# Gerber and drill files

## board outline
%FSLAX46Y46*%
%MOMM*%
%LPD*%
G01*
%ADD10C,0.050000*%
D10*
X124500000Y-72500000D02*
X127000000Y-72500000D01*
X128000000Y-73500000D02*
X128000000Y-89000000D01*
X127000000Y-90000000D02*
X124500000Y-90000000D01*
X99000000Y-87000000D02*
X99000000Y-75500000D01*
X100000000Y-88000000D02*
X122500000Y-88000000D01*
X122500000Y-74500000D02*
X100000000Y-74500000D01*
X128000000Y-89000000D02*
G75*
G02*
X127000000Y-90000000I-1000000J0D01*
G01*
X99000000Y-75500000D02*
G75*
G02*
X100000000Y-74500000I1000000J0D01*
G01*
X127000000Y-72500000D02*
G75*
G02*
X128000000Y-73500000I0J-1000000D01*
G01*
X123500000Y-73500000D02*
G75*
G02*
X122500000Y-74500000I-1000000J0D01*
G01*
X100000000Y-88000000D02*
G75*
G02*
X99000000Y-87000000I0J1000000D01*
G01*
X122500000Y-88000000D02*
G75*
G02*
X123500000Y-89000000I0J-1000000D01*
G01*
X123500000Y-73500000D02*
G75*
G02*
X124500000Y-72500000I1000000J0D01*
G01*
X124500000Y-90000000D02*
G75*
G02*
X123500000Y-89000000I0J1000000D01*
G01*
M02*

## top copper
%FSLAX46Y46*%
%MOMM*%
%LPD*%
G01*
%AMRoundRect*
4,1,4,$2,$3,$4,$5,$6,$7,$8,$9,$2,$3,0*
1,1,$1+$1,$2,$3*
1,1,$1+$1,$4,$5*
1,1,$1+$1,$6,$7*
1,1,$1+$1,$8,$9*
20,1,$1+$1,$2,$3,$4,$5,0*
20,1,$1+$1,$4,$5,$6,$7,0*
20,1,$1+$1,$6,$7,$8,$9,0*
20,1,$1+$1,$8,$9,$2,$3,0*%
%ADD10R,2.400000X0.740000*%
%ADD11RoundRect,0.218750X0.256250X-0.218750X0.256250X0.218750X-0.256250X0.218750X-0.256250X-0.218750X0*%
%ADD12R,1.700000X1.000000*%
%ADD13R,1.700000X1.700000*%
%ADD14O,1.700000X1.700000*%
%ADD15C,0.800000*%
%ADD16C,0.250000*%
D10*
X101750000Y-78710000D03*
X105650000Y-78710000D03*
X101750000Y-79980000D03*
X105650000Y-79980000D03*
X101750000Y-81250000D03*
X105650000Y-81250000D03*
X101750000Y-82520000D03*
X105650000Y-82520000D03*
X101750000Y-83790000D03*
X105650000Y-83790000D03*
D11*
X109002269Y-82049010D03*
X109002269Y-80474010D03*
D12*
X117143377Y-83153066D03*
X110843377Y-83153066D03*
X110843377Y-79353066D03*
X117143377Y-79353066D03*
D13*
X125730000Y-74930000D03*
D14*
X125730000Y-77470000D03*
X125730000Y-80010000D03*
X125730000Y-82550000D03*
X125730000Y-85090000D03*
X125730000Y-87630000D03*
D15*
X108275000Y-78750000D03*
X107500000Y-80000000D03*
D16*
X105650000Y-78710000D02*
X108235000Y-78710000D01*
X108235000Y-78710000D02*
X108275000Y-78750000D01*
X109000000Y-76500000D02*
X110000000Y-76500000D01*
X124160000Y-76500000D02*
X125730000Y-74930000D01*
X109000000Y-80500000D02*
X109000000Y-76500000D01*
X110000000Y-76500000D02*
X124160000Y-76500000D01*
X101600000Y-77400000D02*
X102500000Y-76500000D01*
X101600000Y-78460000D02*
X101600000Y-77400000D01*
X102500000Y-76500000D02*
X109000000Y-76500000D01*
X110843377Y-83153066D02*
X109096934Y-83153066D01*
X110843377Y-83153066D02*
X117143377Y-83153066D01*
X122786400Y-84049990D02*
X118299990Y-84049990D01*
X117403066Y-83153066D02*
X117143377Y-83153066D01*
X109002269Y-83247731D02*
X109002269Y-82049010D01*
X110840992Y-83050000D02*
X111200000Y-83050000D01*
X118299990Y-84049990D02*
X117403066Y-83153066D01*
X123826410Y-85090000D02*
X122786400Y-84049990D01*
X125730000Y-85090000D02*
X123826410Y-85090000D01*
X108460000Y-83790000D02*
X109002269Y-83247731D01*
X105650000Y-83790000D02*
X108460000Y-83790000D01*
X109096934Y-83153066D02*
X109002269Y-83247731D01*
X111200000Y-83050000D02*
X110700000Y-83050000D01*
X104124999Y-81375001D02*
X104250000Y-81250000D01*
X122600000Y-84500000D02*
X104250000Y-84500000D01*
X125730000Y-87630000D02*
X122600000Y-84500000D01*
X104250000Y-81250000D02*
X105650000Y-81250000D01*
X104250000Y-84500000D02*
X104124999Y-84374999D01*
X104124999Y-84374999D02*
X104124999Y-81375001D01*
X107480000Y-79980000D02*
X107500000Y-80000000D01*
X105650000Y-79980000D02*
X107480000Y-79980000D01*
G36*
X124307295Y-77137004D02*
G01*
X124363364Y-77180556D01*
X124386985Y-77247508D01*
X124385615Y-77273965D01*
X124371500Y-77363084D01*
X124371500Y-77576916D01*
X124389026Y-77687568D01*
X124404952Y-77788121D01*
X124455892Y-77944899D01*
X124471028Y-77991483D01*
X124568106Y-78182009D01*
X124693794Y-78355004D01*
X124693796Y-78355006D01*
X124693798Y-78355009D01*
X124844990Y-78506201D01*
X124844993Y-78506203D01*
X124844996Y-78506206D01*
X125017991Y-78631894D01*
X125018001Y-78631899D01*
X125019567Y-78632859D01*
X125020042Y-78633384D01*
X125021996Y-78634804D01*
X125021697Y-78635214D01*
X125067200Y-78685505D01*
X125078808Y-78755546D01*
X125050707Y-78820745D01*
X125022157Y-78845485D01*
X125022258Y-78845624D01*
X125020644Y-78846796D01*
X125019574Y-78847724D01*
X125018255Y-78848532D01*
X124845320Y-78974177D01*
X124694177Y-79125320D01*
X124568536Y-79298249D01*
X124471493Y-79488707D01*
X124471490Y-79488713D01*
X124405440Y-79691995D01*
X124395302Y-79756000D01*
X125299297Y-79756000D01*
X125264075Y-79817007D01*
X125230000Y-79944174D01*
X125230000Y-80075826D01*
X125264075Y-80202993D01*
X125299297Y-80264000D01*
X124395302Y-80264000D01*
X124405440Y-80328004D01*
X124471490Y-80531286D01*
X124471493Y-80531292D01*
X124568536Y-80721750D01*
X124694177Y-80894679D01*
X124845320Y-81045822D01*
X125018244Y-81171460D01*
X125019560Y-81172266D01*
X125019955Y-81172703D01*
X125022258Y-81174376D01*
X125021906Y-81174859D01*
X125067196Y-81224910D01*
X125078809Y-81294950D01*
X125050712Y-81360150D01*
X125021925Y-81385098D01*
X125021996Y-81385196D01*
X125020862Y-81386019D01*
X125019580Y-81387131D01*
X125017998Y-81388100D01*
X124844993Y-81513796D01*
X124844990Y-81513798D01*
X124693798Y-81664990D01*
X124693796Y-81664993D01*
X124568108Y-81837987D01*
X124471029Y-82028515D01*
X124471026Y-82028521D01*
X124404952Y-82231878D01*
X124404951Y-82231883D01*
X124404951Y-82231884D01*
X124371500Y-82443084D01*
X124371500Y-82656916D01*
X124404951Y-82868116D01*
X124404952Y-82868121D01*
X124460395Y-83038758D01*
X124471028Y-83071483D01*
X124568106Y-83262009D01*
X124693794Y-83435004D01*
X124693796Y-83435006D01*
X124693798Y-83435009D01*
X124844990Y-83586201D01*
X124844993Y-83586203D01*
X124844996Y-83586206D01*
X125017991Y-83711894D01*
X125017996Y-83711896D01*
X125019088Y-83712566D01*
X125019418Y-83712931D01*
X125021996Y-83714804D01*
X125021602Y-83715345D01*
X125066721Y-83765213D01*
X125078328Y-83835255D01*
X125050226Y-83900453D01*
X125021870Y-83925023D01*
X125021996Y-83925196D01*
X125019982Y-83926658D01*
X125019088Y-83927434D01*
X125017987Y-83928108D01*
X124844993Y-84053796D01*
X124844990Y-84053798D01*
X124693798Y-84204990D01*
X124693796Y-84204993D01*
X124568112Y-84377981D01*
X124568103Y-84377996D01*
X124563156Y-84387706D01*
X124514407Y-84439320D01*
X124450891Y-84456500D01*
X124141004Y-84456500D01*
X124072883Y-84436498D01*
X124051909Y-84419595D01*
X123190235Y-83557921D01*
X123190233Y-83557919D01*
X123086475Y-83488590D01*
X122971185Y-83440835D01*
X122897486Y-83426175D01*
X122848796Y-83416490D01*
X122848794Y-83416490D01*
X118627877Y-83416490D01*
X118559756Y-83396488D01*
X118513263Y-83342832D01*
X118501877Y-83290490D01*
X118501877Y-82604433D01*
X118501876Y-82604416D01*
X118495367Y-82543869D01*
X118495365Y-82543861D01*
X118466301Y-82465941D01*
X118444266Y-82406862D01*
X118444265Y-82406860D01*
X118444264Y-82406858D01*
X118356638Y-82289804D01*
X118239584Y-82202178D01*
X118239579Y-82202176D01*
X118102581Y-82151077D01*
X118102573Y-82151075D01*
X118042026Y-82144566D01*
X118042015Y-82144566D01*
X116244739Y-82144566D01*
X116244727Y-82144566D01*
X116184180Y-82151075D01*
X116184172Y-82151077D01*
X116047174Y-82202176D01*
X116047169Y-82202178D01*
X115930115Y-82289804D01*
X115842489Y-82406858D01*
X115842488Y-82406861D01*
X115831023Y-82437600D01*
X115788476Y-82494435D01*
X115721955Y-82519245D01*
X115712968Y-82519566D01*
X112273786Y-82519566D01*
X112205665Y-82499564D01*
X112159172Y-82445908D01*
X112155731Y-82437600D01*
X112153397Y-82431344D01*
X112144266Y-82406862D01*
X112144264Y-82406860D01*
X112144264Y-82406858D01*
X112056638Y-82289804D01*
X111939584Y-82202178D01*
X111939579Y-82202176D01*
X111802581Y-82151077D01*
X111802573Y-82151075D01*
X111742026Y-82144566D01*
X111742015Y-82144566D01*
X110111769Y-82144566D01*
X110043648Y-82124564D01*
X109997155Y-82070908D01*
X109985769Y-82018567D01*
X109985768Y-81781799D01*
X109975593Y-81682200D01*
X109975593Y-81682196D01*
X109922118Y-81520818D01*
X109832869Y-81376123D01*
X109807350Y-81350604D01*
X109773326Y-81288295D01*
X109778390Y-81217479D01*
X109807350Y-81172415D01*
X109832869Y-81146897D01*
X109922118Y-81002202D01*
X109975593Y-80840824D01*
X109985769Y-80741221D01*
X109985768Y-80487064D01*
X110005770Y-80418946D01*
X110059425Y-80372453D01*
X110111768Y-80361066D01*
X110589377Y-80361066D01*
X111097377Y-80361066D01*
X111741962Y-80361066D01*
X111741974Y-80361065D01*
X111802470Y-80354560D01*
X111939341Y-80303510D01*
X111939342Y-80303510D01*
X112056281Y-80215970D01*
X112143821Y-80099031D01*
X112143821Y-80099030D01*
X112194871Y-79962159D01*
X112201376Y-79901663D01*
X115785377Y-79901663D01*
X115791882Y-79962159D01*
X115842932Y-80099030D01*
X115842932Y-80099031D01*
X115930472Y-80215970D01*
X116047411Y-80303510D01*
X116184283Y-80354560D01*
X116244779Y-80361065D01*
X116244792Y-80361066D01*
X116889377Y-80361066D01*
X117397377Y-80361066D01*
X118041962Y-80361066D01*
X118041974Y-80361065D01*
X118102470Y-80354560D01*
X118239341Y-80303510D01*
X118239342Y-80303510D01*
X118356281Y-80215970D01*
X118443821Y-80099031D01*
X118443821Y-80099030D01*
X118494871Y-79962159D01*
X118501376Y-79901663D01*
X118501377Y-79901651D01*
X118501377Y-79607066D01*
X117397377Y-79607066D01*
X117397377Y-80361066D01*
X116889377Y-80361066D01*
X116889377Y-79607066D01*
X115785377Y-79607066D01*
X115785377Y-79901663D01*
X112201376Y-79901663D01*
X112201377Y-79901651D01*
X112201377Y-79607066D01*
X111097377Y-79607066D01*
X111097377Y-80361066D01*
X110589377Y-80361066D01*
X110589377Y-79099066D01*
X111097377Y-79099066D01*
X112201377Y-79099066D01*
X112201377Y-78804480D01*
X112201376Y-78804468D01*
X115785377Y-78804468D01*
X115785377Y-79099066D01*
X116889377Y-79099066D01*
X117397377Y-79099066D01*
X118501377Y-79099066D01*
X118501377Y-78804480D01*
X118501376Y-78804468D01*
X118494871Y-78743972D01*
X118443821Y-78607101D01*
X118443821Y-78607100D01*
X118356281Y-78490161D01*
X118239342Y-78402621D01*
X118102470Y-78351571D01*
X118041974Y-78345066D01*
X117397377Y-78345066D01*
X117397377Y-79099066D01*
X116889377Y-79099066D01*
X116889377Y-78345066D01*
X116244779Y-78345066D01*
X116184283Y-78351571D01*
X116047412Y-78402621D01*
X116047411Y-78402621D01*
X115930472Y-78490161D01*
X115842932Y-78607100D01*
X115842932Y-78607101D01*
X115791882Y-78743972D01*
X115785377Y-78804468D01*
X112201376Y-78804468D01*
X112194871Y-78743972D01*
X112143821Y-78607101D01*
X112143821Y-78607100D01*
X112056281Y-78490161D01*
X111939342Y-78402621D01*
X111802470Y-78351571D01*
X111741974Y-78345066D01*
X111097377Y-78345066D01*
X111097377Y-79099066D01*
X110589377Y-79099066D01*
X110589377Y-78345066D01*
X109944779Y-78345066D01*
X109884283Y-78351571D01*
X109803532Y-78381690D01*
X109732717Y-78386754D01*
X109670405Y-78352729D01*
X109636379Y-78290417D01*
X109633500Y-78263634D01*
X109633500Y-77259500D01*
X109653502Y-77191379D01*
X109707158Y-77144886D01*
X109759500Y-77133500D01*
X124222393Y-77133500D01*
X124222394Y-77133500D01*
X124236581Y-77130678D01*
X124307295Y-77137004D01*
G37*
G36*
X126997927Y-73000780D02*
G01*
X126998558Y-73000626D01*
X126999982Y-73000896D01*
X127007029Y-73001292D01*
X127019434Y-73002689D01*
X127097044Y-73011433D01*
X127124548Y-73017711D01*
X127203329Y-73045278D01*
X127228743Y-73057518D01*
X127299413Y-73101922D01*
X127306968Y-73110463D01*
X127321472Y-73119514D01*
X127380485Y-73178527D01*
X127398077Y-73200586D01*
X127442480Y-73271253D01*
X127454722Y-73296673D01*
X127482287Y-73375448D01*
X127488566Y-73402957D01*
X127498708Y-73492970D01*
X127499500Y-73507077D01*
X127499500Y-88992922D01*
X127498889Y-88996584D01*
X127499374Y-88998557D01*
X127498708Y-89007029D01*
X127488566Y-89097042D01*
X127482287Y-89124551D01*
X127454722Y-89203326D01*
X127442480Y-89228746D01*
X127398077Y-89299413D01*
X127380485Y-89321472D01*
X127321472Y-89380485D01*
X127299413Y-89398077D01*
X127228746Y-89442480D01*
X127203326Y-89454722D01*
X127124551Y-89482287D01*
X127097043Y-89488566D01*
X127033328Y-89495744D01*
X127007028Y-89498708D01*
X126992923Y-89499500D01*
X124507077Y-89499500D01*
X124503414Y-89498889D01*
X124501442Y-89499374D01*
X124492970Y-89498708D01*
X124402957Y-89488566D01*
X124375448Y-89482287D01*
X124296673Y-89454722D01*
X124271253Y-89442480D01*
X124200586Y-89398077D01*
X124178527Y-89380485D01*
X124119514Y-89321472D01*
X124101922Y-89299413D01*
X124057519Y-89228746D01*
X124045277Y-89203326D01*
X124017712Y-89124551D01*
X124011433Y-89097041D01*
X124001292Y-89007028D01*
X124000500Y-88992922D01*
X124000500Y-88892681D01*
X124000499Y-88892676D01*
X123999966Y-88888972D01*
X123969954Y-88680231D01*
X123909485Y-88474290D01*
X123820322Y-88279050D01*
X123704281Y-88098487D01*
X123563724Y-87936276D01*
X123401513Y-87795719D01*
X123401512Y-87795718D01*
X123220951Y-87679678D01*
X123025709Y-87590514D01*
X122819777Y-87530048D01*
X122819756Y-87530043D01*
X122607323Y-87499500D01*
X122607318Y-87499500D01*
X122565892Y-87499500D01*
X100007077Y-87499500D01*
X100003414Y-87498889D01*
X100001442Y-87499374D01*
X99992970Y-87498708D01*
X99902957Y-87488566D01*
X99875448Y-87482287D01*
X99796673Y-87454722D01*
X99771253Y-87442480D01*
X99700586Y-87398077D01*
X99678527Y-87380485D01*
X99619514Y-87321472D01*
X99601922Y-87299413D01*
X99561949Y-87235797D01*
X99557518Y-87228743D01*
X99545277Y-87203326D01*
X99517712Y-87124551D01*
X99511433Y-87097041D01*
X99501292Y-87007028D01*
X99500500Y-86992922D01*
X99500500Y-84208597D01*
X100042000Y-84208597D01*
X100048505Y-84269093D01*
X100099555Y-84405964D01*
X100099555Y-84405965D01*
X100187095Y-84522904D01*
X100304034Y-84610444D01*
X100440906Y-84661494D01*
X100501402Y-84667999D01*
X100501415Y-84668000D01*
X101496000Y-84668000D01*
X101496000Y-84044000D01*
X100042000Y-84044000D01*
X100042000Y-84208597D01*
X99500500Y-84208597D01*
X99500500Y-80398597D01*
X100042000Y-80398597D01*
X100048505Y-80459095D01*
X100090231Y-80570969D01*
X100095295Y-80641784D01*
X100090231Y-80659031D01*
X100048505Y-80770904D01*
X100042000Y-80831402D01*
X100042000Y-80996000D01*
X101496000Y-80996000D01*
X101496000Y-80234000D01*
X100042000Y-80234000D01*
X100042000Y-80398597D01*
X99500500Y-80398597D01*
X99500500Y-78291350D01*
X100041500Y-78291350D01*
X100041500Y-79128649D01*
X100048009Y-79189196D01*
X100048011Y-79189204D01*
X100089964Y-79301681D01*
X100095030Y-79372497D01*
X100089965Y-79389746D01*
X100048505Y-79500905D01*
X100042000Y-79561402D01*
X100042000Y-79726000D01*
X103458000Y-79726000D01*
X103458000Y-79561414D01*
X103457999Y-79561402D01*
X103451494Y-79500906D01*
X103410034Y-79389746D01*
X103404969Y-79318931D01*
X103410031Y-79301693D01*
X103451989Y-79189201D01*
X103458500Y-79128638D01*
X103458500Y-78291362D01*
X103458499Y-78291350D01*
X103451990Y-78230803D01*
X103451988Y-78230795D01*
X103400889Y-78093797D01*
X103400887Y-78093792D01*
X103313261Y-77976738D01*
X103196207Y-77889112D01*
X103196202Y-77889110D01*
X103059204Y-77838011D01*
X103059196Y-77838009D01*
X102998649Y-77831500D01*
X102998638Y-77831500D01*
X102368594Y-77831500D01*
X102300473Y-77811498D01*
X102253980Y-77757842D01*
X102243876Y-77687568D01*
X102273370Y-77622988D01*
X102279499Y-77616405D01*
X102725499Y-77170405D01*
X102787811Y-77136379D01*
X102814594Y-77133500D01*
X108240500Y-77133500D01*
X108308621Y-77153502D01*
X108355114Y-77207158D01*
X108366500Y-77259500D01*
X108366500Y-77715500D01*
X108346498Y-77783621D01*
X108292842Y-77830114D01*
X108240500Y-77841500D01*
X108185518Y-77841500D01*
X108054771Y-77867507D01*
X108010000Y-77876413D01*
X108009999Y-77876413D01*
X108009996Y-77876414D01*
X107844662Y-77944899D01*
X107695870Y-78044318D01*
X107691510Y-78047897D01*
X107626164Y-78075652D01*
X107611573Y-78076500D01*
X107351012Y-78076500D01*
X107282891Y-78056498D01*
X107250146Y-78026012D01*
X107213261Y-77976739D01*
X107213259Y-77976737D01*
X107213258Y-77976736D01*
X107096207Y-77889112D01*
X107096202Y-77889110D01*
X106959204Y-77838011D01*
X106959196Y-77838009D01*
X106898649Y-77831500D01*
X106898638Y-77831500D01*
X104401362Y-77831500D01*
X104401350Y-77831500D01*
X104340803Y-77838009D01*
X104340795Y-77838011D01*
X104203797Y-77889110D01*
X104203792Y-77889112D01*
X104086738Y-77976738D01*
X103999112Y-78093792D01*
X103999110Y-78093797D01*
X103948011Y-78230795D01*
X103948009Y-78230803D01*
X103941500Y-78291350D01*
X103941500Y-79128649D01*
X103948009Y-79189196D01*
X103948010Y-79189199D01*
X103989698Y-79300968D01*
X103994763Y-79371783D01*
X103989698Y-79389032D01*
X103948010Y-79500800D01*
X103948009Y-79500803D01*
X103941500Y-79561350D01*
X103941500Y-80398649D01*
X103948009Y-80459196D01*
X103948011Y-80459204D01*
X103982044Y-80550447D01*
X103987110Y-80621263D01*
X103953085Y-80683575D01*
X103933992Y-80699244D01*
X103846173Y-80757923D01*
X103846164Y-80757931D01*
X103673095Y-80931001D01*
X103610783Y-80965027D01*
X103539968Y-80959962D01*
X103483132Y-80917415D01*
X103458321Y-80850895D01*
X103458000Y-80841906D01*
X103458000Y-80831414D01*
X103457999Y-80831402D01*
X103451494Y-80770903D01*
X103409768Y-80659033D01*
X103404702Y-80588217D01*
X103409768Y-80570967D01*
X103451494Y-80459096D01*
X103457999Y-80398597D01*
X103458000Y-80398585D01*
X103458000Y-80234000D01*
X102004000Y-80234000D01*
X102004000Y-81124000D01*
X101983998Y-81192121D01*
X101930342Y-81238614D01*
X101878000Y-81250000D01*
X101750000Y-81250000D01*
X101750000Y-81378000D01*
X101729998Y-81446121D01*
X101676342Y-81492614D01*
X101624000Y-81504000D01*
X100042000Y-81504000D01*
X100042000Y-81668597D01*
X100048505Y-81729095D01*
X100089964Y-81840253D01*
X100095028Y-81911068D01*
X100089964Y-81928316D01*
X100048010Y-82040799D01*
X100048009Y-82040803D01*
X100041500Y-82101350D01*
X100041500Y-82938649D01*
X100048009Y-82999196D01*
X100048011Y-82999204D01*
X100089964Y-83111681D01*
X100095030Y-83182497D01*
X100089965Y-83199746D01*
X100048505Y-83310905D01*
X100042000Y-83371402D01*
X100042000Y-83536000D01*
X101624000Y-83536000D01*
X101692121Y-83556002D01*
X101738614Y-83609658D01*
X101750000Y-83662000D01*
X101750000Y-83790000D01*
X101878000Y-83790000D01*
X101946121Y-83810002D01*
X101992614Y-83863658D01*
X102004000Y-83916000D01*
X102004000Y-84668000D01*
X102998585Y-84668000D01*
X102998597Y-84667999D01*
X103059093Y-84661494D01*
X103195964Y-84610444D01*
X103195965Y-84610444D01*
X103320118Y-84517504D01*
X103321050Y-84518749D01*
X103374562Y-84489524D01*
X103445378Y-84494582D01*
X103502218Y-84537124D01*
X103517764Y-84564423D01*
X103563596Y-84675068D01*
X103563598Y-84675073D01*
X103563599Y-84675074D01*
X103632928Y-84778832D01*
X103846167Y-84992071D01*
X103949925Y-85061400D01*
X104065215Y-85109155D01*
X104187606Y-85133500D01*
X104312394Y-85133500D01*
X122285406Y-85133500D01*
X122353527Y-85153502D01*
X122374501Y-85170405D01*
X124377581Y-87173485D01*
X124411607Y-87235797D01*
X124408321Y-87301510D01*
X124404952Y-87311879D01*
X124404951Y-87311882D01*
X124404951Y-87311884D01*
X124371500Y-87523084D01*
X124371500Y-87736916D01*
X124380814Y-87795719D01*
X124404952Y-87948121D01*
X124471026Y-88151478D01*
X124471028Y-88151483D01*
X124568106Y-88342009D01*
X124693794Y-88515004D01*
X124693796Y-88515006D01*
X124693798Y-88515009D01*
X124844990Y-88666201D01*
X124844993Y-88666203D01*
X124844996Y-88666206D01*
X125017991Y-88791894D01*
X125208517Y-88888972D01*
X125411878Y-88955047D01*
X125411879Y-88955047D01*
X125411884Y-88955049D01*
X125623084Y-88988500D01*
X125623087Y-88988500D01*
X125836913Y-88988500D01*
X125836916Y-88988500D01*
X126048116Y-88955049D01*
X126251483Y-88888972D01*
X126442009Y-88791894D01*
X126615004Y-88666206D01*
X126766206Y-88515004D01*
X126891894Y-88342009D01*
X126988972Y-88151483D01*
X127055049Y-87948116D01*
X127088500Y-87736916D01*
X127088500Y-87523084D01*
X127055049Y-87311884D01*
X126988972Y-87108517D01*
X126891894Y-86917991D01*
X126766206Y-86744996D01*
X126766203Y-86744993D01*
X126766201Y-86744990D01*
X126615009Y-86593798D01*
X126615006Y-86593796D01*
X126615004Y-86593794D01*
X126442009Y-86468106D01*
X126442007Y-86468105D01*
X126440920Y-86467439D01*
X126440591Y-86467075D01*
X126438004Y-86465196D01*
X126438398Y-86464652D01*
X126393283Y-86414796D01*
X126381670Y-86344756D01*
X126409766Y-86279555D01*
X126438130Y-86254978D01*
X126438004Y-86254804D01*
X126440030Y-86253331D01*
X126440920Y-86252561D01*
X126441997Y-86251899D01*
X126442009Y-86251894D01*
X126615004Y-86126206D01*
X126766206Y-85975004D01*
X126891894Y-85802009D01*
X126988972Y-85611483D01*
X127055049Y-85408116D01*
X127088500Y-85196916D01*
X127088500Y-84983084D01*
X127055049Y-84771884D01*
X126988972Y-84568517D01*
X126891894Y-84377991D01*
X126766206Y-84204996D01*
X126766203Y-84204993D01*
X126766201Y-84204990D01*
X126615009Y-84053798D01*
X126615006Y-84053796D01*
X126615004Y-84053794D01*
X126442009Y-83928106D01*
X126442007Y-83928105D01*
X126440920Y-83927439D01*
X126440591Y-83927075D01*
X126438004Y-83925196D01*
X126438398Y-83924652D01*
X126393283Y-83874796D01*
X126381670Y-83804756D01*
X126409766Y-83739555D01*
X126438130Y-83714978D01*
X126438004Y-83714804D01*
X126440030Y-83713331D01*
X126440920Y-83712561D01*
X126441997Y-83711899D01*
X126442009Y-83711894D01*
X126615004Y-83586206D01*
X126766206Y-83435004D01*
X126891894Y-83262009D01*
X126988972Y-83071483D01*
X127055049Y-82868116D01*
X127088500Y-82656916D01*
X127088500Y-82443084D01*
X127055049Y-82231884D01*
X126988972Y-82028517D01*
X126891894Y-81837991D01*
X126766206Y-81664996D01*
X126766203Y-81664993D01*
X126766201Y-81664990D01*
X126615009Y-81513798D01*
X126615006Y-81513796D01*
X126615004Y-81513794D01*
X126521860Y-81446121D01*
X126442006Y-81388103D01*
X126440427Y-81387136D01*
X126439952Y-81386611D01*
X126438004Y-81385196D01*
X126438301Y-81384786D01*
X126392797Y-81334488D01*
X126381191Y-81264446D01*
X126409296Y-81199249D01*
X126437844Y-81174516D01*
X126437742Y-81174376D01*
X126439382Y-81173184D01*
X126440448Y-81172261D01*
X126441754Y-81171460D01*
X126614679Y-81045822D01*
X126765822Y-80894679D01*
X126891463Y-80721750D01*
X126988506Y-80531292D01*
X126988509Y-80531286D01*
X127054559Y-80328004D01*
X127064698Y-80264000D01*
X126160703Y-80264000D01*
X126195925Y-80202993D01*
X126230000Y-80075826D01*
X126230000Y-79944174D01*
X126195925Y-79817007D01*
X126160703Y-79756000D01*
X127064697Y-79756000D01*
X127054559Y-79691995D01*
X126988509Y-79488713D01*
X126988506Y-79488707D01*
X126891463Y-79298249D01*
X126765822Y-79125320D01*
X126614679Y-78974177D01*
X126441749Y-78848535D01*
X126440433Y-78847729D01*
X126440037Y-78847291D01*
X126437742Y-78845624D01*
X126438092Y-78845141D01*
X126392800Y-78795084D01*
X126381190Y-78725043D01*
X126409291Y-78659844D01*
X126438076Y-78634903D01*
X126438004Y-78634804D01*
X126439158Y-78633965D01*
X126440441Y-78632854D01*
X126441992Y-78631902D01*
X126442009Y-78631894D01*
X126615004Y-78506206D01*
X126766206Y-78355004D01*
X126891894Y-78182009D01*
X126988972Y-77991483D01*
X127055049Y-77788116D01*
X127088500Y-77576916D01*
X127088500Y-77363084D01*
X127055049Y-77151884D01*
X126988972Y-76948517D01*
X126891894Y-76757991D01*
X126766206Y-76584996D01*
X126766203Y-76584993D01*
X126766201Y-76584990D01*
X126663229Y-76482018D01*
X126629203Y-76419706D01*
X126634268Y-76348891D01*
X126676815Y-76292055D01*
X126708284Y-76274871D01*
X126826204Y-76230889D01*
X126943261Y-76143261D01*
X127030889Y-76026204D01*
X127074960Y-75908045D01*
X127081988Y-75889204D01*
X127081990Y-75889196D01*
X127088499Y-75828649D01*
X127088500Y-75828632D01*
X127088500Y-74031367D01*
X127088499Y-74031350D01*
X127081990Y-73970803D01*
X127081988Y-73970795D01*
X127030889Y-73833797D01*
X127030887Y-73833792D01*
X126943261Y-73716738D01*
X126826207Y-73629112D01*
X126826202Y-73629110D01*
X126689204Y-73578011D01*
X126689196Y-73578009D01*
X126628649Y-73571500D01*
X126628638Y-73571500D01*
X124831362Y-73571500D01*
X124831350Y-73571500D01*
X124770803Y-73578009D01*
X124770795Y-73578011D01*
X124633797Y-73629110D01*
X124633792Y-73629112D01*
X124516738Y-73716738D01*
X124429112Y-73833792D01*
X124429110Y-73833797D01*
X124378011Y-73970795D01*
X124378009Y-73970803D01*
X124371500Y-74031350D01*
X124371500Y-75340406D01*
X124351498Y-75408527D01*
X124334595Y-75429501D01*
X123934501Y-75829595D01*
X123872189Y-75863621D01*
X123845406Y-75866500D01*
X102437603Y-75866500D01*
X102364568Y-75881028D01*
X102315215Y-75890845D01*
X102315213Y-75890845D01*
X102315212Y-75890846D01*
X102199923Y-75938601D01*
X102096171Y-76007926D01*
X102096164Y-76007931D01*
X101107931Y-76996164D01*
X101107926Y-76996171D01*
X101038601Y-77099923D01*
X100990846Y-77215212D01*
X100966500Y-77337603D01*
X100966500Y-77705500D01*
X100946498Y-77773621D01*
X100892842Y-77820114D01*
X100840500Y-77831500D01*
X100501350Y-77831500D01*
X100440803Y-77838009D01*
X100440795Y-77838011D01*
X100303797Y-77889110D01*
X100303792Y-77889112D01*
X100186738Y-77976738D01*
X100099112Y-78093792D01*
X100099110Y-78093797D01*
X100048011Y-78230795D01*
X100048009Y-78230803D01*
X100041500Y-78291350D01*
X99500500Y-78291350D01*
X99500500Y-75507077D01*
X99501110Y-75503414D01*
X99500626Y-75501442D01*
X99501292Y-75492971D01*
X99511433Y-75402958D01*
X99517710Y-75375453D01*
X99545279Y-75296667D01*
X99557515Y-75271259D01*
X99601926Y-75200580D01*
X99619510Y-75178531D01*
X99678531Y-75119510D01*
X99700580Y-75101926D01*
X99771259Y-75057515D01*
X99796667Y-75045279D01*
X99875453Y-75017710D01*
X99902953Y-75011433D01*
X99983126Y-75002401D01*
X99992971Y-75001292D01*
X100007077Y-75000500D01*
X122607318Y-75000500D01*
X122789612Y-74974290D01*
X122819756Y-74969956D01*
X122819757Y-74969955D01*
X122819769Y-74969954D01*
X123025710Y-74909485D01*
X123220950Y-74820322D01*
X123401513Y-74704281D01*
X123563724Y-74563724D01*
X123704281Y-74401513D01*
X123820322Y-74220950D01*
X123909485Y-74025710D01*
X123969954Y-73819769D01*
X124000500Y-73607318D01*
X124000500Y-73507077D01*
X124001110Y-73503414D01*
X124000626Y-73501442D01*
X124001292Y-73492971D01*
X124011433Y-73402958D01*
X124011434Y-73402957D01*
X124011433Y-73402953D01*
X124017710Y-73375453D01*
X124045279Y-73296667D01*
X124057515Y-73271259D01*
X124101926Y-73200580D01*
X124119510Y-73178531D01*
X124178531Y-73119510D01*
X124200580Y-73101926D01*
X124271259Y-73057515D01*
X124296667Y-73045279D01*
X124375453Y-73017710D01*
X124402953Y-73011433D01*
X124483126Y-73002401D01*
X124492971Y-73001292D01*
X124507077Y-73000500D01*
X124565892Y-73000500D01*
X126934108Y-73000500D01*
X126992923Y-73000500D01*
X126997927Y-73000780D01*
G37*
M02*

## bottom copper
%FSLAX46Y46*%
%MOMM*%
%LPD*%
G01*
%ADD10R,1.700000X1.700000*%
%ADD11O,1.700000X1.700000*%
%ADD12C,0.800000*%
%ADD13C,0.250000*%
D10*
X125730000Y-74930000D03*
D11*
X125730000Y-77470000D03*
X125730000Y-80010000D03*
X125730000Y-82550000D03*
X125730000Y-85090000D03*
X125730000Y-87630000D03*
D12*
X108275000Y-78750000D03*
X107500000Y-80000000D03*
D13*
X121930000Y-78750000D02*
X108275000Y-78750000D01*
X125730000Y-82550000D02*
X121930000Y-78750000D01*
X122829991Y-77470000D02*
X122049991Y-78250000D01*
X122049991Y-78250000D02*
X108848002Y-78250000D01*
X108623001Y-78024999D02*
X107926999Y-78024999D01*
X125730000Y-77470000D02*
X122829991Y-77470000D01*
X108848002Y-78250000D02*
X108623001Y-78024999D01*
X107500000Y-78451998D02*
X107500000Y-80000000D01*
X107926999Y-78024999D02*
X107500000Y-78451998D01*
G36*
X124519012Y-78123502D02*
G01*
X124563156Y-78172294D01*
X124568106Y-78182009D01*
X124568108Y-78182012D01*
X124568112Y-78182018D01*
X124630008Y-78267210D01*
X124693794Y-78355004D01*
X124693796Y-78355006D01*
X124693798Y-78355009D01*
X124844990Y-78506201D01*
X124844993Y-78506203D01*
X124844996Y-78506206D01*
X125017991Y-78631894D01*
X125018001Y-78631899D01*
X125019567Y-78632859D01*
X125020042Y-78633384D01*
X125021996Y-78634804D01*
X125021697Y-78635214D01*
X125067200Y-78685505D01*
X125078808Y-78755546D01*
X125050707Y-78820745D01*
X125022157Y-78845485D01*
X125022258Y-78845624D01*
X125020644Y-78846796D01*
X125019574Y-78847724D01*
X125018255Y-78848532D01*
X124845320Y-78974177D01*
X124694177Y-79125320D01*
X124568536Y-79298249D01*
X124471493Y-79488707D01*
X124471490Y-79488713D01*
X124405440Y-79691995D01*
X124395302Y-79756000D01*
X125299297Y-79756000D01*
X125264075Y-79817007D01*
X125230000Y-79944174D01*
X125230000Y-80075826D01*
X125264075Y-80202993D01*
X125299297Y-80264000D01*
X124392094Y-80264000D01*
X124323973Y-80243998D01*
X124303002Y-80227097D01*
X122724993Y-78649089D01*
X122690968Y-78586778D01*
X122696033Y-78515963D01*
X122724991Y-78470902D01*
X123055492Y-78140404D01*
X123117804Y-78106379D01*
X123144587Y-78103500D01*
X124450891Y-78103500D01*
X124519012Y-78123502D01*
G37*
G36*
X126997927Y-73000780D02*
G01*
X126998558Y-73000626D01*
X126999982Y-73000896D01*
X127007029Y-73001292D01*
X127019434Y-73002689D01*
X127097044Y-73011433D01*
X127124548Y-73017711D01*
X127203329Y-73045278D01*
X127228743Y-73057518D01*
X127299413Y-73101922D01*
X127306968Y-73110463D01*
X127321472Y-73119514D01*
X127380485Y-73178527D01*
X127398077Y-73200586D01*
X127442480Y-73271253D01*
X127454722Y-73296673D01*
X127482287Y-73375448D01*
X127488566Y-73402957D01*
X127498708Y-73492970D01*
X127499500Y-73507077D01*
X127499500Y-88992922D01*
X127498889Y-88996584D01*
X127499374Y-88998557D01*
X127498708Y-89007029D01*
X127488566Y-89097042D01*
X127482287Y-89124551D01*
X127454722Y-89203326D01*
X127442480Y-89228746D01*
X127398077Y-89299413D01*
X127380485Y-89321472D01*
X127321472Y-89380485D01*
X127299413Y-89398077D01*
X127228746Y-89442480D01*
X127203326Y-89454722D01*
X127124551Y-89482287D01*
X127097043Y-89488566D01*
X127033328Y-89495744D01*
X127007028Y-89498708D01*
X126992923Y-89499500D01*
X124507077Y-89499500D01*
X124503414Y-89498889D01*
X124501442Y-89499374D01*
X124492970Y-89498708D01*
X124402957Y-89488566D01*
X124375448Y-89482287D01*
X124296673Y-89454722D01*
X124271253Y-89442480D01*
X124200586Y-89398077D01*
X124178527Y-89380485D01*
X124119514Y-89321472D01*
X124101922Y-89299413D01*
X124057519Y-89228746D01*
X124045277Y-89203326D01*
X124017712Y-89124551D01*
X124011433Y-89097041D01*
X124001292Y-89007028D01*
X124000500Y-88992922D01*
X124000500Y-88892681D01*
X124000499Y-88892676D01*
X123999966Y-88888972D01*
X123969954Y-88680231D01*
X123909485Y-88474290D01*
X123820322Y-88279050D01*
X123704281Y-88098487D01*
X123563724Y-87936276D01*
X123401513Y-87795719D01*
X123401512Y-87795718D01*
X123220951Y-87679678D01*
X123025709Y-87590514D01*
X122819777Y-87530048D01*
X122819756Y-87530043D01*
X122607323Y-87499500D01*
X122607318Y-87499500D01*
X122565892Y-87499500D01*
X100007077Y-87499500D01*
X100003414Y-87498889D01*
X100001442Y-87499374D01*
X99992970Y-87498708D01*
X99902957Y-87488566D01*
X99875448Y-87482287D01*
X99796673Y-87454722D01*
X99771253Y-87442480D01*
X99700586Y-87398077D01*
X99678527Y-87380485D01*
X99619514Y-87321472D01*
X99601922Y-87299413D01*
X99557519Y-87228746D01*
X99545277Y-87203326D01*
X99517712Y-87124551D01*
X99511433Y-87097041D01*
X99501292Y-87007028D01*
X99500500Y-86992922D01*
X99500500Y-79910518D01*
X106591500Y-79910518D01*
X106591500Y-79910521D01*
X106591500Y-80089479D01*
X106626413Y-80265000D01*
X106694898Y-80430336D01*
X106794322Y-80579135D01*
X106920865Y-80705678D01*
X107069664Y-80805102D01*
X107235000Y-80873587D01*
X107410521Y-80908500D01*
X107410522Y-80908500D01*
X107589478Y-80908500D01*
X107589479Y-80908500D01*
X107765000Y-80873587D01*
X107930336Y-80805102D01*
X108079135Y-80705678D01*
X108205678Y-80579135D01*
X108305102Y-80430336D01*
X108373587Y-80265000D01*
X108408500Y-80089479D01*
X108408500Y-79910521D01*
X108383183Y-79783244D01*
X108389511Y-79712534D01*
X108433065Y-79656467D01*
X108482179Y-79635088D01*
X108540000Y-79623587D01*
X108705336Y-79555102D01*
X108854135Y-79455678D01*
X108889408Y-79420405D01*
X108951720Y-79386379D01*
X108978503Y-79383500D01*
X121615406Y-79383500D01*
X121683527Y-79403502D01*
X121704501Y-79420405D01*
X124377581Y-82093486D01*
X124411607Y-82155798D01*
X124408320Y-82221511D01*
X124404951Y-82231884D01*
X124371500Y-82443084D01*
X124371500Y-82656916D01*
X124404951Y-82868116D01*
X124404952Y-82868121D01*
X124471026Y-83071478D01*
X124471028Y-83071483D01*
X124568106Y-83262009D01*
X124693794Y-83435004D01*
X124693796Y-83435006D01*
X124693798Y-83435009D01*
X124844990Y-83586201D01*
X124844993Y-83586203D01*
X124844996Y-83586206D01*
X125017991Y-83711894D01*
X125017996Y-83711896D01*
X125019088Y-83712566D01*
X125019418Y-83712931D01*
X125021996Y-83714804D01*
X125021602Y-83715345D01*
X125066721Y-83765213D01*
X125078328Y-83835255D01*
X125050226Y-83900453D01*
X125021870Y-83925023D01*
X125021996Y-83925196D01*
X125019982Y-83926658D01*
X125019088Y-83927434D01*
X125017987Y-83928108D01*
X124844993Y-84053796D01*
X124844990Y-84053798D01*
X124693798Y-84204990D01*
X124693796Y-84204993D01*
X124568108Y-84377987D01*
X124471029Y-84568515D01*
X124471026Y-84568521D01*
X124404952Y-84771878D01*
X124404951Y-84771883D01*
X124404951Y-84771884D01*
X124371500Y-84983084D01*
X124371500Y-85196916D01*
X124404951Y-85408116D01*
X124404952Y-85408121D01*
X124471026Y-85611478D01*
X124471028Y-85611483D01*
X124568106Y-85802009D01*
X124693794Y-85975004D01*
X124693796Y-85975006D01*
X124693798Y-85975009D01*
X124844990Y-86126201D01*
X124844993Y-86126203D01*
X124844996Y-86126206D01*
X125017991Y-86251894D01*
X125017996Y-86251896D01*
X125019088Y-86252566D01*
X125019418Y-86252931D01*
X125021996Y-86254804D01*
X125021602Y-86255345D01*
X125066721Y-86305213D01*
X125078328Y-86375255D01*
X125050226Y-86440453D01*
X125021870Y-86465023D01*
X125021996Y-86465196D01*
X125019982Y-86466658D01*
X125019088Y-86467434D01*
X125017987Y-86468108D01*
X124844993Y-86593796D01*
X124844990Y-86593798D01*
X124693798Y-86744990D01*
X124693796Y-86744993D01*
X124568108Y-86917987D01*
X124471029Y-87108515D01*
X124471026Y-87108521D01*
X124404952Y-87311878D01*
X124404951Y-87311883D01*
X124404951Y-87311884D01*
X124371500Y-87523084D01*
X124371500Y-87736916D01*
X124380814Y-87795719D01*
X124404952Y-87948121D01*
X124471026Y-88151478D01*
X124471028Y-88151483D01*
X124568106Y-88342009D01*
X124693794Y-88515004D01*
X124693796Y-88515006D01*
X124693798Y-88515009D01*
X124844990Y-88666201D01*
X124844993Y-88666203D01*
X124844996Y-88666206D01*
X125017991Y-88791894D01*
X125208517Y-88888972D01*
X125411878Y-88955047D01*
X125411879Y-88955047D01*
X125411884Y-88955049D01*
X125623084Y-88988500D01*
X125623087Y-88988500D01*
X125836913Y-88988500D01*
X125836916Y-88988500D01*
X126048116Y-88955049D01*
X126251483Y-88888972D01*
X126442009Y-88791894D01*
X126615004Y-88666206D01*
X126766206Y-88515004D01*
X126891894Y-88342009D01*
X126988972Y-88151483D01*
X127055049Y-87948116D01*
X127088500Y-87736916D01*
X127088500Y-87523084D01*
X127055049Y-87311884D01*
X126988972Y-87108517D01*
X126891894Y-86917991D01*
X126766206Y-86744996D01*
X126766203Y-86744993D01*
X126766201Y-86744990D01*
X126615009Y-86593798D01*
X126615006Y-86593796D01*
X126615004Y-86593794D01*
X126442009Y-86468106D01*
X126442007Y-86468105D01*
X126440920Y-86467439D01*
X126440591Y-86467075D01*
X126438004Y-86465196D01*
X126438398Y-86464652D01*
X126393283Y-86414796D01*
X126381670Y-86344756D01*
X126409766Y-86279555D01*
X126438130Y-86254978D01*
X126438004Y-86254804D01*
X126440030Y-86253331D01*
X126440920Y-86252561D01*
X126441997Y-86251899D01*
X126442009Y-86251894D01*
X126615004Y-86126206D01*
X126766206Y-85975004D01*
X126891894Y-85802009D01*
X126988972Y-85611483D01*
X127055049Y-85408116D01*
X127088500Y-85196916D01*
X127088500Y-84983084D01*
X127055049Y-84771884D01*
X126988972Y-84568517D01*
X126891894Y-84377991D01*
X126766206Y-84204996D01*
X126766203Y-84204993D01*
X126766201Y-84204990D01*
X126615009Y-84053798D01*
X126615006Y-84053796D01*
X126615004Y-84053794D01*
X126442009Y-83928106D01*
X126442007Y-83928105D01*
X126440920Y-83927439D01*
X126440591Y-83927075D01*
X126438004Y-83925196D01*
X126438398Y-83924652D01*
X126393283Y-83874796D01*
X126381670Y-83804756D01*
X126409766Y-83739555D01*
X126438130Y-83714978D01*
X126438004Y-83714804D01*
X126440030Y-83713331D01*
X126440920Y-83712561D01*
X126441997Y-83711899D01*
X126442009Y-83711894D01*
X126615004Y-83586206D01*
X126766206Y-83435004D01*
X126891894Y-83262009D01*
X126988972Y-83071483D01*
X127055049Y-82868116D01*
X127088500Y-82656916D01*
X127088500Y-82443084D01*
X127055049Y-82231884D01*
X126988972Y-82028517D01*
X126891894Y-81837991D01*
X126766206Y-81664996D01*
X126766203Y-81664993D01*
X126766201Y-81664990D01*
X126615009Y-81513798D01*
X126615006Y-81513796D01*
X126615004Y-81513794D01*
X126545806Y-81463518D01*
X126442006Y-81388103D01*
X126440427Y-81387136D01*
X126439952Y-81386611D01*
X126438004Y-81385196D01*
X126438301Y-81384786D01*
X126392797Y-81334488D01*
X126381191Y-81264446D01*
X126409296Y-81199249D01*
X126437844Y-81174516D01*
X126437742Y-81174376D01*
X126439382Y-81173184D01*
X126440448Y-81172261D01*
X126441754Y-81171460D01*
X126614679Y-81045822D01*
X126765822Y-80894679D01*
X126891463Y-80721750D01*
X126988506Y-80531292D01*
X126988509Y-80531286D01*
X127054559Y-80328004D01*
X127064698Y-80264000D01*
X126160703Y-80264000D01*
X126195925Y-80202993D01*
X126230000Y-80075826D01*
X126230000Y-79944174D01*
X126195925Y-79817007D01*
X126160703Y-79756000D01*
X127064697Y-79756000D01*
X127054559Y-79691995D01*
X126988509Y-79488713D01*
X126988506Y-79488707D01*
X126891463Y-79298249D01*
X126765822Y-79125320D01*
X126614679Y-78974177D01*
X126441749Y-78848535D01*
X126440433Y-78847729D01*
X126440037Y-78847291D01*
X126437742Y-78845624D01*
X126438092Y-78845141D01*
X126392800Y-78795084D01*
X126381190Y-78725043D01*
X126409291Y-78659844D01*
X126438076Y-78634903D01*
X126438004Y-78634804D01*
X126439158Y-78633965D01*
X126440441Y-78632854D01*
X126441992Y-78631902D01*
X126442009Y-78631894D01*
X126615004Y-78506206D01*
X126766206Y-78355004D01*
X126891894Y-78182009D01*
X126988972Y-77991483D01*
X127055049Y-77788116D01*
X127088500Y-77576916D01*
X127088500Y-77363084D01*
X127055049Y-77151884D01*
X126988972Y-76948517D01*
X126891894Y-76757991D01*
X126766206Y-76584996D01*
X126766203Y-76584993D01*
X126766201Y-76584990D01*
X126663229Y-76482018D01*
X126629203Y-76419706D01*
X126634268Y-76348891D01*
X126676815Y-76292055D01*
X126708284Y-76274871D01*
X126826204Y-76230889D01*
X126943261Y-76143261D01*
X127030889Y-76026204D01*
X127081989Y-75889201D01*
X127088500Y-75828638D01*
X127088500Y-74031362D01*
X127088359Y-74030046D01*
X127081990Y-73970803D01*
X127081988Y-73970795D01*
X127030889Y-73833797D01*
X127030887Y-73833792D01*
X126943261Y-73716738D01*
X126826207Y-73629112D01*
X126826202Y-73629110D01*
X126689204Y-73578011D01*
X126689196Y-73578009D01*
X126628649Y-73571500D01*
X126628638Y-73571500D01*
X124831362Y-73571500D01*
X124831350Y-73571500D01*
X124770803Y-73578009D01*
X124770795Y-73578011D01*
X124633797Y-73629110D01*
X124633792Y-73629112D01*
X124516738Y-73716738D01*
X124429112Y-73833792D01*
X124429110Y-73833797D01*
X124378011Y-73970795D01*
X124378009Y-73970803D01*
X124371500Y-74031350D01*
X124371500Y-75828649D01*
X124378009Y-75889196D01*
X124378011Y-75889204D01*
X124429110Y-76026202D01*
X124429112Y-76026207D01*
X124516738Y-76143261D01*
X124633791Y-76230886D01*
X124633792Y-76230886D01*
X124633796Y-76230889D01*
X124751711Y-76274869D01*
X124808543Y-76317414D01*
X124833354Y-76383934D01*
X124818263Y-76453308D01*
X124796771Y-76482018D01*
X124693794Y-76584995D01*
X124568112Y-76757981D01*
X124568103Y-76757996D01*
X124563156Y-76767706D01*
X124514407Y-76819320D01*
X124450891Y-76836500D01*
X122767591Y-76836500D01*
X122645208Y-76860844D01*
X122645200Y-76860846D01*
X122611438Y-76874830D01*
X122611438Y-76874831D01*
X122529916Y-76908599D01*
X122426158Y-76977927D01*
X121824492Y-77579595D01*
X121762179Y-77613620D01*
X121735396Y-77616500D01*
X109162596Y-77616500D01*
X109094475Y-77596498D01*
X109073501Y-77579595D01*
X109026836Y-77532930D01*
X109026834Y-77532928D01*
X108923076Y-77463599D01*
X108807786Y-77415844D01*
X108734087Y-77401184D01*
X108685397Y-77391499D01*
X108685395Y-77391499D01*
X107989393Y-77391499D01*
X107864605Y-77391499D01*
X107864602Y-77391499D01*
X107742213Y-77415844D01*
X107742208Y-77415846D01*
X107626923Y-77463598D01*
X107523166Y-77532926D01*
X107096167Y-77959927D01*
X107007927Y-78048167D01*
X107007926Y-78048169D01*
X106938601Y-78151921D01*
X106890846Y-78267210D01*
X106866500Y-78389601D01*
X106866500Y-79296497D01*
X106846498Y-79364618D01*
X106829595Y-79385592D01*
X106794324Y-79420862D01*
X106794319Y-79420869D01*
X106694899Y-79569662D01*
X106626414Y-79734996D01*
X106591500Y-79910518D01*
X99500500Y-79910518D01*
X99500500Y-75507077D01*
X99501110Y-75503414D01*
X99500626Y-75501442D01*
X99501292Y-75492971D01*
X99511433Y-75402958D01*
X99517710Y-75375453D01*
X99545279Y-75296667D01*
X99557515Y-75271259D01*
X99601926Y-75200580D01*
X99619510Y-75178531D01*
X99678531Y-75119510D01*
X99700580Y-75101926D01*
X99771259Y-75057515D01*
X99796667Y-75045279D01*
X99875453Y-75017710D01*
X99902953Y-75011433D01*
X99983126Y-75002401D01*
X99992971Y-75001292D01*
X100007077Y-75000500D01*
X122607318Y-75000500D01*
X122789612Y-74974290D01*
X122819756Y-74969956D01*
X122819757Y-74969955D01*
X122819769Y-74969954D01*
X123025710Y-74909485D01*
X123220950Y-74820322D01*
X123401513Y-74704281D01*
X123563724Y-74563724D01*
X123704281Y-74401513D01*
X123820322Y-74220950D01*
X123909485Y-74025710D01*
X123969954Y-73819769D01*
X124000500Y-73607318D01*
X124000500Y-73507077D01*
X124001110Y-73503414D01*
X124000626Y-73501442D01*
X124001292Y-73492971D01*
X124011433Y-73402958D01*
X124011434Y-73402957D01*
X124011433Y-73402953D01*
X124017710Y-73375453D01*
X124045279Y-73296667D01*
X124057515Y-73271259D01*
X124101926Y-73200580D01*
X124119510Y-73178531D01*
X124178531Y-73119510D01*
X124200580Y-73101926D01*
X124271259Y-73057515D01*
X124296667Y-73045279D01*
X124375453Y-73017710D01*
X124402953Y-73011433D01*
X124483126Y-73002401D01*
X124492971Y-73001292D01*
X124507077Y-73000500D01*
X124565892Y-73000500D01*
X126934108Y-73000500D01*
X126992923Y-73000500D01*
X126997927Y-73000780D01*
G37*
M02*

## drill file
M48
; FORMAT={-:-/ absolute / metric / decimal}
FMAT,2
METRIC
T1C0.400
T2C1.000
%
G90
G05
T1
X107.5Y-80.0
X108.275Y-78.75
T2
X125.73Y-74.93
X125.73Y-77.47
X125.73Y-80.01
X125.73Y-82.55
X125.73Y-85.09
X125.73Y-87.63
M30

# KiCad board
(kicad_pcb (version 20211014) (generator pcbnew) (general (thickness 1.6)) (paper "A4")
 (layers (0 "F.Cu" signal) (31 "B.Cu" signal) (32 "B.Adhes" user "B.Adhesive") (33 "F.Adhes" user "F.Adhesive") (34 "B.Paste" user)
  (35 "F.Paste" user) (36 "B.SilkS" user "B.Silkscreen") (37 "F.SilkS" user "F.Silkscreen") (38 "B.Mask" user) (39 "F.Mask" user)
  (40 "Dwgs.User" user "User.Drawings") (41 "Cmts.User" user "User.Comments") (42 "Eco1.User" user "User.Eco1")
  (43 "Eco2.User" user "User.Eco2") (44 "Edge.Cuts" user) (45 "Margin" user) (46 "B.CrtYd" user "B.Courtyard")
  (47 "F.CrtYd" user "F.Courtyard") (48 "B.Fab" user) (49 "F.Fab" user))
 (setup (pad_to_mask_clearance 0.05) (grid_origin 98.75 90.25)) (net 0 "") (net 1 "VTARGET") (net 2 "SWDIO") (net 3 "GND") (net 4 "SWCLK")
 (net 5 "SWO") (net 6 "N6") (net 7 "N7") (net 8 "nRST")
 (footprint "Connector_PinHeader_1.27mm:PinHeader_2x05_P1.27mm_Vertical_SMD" (layer "F.Cu") (at 103.7 81.25)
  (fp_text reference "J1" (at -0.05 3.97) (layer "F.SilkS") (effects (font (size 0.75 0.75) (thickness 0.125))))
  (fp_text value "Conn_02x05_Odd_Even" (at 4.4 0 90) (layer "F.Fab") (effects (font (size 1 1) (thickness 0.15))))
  (pad "1" smd rect locked (at -1.95 -2.54) (size 2.4 0.74) (layers "F.Cu" "F.Paste" "F.Mask") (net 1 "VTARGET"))
  (pad "2" smd rect locked (at 1.95 -2.54) (size 2.4 0.74) (layers "F.Cu" "F.Paste" "F.Mask") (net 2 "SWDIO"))
  (pad "3" smd rect locked (at -1.95 -1.27) (size 2.4 0.74) (layers "F.Cu" "F.Paste" "F.Mask") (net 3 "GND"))
  (pad "4" smd rect locked (at 1.95 -1.27) (size 2.4 0.74) (layers "F.Cu" "F.Paste" "F.Mask") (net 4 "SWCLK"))
  (pad "5" smd rect locked (at -1.95 0) (size 2.4 0.74) (layers "F.Cu" "F.Paste" "F.Mask") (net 3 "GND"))
  (pad "6" smd rect locked (at 1.95 0) (size 2.4 0.74) (layers "F.Cu" "F.Paste" "F.Mask") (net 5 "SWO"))
  (pad "7" smd rect locked (at -1.95 1.27) (size 2.4 0.74) (layers "F.Cu" "F.Paste" "F.Mask") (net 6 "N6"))
  (pad "8" smd rect locked (at 1.95 1.27) (size 2.4 0.74) (layers "F.Cu" "F.Paste" "F.Mask") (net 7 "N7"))
  (pad "9" smd rect locked (at -1.95 2.54) (size 2.4 0.74) (layers "F.Cu" "F.Paste" "F.Mask") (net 3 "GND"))
  (pad "10" smd rect locked (at 1.95 2.54) (size 2.4 0.74) (layers "F.Cu" "F.Paste" "F.Mask") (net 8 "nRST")))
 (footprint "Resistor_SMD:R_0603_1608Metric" (layer "F.Cu") (at 109.002269 81.26151 90)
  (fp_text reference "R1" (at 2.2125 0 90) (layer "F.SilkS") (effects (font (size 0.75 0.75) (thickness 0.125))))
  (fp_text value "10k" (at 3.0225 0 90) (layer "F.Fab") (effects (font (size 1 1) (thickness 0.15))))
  (pad "1" smd roundrect locked (at -0.7875 0 90) (size 0.875 0.95) (layers "F.Cu" "F.Paste" "F.Mask") (roundrect_rratio 0.25)
   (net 8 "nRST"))
  (pad "2" smd roundrect locked (at 0.7875 0 90) (size 0.875 0.95) (layers "F.Cu" "F.Paste" "F.Mask") (roundrect_rratio 0.25)
   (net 1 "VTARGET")))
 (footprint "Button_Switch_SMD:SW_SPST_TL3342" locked (layer "F.Cu") (at 113.993377 81.253066 180)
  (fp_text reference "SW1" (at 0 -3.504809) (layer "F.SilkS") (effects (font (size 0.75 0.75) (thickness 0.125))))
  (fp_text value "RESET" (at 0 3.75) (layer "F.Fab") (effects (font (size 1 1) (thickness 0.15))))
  (pad "1" smd rect locked (at -3.15 -1.9 180) (size 1.7 1) (layers "F.Cu" "F.Paste" "F.Mask") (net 8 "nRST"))
  (pad "1" smd rect locked (at 3.15 -1.9 180) (size 1.7 1) (layers "F.Cu" "F.Paste" "F.Mask") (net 8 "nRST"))
  (pad "2" smd rect locked (at 3.15 1.9 180) (size 1.7 1) (layers "F.Cu" "F.Paste" "F.Mask") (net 3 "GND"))
  (pad "2" smd rect locked (at -3.15 1.9 180) (size 1.7 1) (layers "F.Cu" "F.Paste" "F.Mask") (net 3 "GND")))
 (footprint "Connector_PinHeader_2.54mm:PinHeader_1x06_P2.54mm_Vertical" (layer "B.Cu") (at 125.73 74.93 180)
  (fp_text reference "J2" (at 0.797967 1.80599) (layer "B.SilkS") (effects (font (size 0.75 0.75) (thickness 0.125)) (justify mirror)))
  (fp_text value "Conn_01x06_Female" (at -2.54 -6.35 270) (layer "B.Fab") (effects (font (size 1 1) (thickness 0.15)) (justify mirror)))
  (pad "1" thru_hole rect locked (at 0 0 180) (size 1.7 1.7) (drill 1) (layers *.Cu *.Mask) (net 1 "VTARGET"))
  (pad "2" thru_hole oval locked (at 0 -2.54 180) (size 1.7 1.7) (drill 1) (layers *.Cu *.Mask) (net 4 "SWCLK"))
  (pad "3" thru_hole oval locked (at 0 -5.08 180) (size 1.7 1.7) (drill 1) (layers *.Cu *.Mask) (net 3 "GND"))
  (pad "4" thru_hole oval locked (at 0 -7.62 180) (size 1.7 1.7) (drill 1) (layers *.Cu *.Mask) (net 2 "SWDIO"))
  (pad "5" thru_hole oval locked (at 0 -10.16 180) (size 1.7 1.7) (drill 1) (layers *.Cu *.Mask) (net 8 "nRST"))
  (pad "6" thru_hole oval locked (at 0 -12.7 180) (size 1.7 1.7) (drill 1) (layers *.Cu *.Mask) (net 5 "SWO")))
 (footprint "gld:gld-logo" (layer "B.Cu") (at 116.45 80.05 180)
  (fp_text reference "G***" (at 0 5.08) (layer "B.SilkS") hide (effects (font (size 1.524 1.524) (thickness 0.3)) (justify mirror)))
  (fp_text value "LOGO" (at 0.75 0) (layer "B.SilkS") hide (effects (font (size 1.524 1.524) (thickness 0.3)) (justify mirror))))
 (gr_line (start 124.5 72.5) (end 127 72.5) (layer "Edge.Cuts") (width 0.05))
 (gr_line (start 128 73.5) (end 128 89) (layer "Edge.Cuts") (width 0.05))
 (gr_line (start 127 90) (end 124.5 90) (layer "Edge.Cuts") (width 0.05))
 (gr_line (start 99 87) (end 99 75.5) (layer "Edge.Cuts") (width 0.05))
 (gr_line (start 100 88) (end 122.5 88) (layer "Edge.Cuts") (width 0.05))
 (gr_line (start 122.5 74.5) (end 100 74.5) (layer "Edge.Cuts") (width 0.05))
 (gr_arc (start 128 89) (mid 127.707107 89.707107) (end 127 90) (layer "Edge.Cuts") (width 0.05))
 (gr_arc (start 99 75.5) (mid 99.292893 74.792893) (end 100 74.5) (layer "Edge.Cuts") (width 0.05))
 (gr_arc (start 127 72.5) (mid 127.707107 72.792893) (end 128 73.5) (layer "Edge.Cuts") (width 0.05))
 (gr_arc (start 123.5 73.5) (mid 123.207107 74.207107) (end 122.5 74.5) (layer "Edge.Cuts") (width 0.05))
 (gr_arc (start 100 88) (mid 99.292893 87.707107) (end 99 87) (layer "Edge.Cuts") (width 0.05))
 (gr_arc (start 122.5 88) (mid 123.207107 88.292893) (end 123.5 89) (layer "Edge.Cuts") (width 0.05))
 (gr_arc (start 123.5 73.5) (mid 123.792893 72.792893) (end 124.5 72.5) (layer "Edge.Cuts") (width 0.05))
 (gr_arc (start 124.5 90) (mid 123.792893 89.707107) (end 123.5 89) (layer "Edge.Cuts") (width 0.05))
 (segment (start 105.65 78.71) (end 108.235 78.71) (width 0.25) (layer "F.Cu") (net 2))
 (segment (start 108.235 78.71) (end 108.275 78.75) (width 0.25) (layer "F.Cu") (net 2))
 (via (at 108.275 78.75) (size 0.8) (drill 0.4) (layers "F.Cu" "B.Cu") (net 2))
 (segment (start 121.93 78.75) (end 108.275 78.75) (width 0.25) (layer "B.Cu") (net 2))
 (segment (start 125.73 82.55) (end 121.93 78.75) (width 0.25) (layer "B.Cu") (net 2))
 (segment (start 109 76.5) (end 110 76.5) (width 0.25) (layer "F.Cu") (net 1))
 (segment (start 124.16 76.5) (end 125.73 74.93) (width 0.25) (layer "F.Cu") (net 1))
 (segment (start 109 80.5) (end 109 76.5) (width 0.25) (layer "F.Cu") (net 1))
 (segment (start 110 76.5) (end 124.16 76.5) (width 0.25) (layer "F.Cu") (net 1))
 (segment (start 101.6 77.4) (end 102.5 76.5) (width 0.25) (layer "F.Cu") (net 1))
 (segment (start 101.6 78.46) (end 101.6 77.4) (width 0.25) (layer "F.Cu") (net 1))
 (segment (start 102.5 76.5) (end 109 76.5) (width 0.25) (layer "F.Cu") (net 1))
 (segment (start 110.843377 83.153066) (end 109.096934 83.153066) (width 0.25) (layer "F.Cu") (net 8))
 (segment (start 110.843377 83.153066) (end 117.143377 83.153066) (width 0.25) (layer "F.Cu") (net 8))
 (segment (start 122.7864 84.04999) (end 118.29999 84.04999) (width 0.25) (layer "F.Cu") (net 8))
 (segment (start 117.403066 83.153066) (end 117.143377 83.153066) (width 0.25) (layer "F.Cu") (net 8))
 (segment (start 109.002269 83.247731) (end 109.002269 82.04901) (width 0.25) (layer "F.Cu") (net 8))
 (segment (start 110.840992 83.05) (end 111.2 83.05) (width 0.25) (layer "F.Cu") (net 8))
 (segment (start 118.29999 84.04999) (end 117.403066 83.153066) (width 0.25) (layer "F.Cu") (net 8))
 (segment (start 123.82641 85.09) (end 122.7864 84.04999) (width 0.25) (layer "F.Cu") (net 8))
 (segment (start 125.73 85.09) (end 123.82641 85.09) (width 0.25) (layer "F.Cu") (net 8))
 (segment (start 108.46 83.79) (end 109.002269 83.247731) (width 0.25) (layer "F.Cu") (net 8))
 (segment (start 105.65 83.79) (end 108.46 83.79) (width 0.25) (layer "F.Cu") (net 8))
 (segment (start 109.096934 83.153066) (end 109.002269 83.247731) (width 0.25) (layer "F.Cu") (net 8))
 (segment (start 111.2 83.05) (end 110.7 83.05) (width 0.25) (layer "F.Cu") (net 8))
 (segment (start 104.124999 81.375001) (end 104.25 81.25) (width 0.25) (layer "F.Cu") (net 5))
 (segment (start 122.6 84.5) (end 104.25 84.5) (width 0.25) (layer "F.Cu") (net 5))
 (segment (start 125.73 87.63) (end 122.6 84.5) (width 0.25) (layer "F.Cu") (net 5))
 (segment (start 104.25 81.25) (end 105.65 81.25) (width 0.25) (layer "F.Cu") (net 5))
 (segment (start 104.25 84.5) (end 104.124999 84.374999) (width 0.25) (layer "F.Cu") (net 5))
 (segment (start 104.124999 84.374999) (end 104.124999 81.375001) (width 0.25) (layer "F.Cu") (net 5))
 (segment (start 107.48 79.98) (end 107.5 80) (width 0.25) (layer "F.Cu") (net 4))
 (segment (start 105.65 79.98) (end 107.48 79.98) (width 0.25) (layer "F.Cu") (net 4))
 (via (at 107.5 80) (size 0.8) (drill 0.4) (layers "F.Cu" "B.Cu") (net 4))
 (segment (start 122.829991 77.47) (end 122.049991 78.25) (width 0.25) (layer "B.Cu") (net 4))
 (segment (start 122.049991 78.25) (end 108.848002 78.25) (width 0.25) (layer "B.Cu") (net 4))
 (segment (start 108.623001 78.024999) (end 107.926999 78.024999) (width 0.25) (layer "B.Cu") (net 4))
 (segment (start 125.73 77.47) (end 122.829991 77.47) (width 0.25) (layer "B.Cu") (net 4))
 (segment (start 108.848002 78.25) (end 108.623001 78.024999) (width 0.25) (layer "B.Cu") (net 4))
 (segment (start 107.5 78.451998) (end 107.5 80) (width 0.25) (layer "B.Cu") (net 4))
 (segment (start 107.926999 78.024999) (end 107.5 78.451998) (width 0.25) (layer "B.Cu") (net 4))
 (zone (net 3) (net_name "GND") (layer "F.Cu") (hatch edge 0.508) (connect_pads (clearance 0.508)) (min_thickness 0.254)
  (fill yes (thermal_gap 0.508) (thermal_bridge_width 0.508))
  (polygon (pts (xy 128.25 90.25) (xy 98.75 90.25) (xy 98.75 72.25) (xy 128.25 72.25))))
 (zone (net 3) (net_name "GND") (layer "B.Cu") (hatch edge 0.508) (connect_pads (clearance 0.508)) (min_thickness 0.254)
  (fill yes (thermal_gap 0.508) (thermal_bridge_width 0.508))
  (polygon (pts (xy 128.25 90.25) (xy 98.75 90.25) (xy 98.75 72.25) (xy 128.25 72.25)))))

